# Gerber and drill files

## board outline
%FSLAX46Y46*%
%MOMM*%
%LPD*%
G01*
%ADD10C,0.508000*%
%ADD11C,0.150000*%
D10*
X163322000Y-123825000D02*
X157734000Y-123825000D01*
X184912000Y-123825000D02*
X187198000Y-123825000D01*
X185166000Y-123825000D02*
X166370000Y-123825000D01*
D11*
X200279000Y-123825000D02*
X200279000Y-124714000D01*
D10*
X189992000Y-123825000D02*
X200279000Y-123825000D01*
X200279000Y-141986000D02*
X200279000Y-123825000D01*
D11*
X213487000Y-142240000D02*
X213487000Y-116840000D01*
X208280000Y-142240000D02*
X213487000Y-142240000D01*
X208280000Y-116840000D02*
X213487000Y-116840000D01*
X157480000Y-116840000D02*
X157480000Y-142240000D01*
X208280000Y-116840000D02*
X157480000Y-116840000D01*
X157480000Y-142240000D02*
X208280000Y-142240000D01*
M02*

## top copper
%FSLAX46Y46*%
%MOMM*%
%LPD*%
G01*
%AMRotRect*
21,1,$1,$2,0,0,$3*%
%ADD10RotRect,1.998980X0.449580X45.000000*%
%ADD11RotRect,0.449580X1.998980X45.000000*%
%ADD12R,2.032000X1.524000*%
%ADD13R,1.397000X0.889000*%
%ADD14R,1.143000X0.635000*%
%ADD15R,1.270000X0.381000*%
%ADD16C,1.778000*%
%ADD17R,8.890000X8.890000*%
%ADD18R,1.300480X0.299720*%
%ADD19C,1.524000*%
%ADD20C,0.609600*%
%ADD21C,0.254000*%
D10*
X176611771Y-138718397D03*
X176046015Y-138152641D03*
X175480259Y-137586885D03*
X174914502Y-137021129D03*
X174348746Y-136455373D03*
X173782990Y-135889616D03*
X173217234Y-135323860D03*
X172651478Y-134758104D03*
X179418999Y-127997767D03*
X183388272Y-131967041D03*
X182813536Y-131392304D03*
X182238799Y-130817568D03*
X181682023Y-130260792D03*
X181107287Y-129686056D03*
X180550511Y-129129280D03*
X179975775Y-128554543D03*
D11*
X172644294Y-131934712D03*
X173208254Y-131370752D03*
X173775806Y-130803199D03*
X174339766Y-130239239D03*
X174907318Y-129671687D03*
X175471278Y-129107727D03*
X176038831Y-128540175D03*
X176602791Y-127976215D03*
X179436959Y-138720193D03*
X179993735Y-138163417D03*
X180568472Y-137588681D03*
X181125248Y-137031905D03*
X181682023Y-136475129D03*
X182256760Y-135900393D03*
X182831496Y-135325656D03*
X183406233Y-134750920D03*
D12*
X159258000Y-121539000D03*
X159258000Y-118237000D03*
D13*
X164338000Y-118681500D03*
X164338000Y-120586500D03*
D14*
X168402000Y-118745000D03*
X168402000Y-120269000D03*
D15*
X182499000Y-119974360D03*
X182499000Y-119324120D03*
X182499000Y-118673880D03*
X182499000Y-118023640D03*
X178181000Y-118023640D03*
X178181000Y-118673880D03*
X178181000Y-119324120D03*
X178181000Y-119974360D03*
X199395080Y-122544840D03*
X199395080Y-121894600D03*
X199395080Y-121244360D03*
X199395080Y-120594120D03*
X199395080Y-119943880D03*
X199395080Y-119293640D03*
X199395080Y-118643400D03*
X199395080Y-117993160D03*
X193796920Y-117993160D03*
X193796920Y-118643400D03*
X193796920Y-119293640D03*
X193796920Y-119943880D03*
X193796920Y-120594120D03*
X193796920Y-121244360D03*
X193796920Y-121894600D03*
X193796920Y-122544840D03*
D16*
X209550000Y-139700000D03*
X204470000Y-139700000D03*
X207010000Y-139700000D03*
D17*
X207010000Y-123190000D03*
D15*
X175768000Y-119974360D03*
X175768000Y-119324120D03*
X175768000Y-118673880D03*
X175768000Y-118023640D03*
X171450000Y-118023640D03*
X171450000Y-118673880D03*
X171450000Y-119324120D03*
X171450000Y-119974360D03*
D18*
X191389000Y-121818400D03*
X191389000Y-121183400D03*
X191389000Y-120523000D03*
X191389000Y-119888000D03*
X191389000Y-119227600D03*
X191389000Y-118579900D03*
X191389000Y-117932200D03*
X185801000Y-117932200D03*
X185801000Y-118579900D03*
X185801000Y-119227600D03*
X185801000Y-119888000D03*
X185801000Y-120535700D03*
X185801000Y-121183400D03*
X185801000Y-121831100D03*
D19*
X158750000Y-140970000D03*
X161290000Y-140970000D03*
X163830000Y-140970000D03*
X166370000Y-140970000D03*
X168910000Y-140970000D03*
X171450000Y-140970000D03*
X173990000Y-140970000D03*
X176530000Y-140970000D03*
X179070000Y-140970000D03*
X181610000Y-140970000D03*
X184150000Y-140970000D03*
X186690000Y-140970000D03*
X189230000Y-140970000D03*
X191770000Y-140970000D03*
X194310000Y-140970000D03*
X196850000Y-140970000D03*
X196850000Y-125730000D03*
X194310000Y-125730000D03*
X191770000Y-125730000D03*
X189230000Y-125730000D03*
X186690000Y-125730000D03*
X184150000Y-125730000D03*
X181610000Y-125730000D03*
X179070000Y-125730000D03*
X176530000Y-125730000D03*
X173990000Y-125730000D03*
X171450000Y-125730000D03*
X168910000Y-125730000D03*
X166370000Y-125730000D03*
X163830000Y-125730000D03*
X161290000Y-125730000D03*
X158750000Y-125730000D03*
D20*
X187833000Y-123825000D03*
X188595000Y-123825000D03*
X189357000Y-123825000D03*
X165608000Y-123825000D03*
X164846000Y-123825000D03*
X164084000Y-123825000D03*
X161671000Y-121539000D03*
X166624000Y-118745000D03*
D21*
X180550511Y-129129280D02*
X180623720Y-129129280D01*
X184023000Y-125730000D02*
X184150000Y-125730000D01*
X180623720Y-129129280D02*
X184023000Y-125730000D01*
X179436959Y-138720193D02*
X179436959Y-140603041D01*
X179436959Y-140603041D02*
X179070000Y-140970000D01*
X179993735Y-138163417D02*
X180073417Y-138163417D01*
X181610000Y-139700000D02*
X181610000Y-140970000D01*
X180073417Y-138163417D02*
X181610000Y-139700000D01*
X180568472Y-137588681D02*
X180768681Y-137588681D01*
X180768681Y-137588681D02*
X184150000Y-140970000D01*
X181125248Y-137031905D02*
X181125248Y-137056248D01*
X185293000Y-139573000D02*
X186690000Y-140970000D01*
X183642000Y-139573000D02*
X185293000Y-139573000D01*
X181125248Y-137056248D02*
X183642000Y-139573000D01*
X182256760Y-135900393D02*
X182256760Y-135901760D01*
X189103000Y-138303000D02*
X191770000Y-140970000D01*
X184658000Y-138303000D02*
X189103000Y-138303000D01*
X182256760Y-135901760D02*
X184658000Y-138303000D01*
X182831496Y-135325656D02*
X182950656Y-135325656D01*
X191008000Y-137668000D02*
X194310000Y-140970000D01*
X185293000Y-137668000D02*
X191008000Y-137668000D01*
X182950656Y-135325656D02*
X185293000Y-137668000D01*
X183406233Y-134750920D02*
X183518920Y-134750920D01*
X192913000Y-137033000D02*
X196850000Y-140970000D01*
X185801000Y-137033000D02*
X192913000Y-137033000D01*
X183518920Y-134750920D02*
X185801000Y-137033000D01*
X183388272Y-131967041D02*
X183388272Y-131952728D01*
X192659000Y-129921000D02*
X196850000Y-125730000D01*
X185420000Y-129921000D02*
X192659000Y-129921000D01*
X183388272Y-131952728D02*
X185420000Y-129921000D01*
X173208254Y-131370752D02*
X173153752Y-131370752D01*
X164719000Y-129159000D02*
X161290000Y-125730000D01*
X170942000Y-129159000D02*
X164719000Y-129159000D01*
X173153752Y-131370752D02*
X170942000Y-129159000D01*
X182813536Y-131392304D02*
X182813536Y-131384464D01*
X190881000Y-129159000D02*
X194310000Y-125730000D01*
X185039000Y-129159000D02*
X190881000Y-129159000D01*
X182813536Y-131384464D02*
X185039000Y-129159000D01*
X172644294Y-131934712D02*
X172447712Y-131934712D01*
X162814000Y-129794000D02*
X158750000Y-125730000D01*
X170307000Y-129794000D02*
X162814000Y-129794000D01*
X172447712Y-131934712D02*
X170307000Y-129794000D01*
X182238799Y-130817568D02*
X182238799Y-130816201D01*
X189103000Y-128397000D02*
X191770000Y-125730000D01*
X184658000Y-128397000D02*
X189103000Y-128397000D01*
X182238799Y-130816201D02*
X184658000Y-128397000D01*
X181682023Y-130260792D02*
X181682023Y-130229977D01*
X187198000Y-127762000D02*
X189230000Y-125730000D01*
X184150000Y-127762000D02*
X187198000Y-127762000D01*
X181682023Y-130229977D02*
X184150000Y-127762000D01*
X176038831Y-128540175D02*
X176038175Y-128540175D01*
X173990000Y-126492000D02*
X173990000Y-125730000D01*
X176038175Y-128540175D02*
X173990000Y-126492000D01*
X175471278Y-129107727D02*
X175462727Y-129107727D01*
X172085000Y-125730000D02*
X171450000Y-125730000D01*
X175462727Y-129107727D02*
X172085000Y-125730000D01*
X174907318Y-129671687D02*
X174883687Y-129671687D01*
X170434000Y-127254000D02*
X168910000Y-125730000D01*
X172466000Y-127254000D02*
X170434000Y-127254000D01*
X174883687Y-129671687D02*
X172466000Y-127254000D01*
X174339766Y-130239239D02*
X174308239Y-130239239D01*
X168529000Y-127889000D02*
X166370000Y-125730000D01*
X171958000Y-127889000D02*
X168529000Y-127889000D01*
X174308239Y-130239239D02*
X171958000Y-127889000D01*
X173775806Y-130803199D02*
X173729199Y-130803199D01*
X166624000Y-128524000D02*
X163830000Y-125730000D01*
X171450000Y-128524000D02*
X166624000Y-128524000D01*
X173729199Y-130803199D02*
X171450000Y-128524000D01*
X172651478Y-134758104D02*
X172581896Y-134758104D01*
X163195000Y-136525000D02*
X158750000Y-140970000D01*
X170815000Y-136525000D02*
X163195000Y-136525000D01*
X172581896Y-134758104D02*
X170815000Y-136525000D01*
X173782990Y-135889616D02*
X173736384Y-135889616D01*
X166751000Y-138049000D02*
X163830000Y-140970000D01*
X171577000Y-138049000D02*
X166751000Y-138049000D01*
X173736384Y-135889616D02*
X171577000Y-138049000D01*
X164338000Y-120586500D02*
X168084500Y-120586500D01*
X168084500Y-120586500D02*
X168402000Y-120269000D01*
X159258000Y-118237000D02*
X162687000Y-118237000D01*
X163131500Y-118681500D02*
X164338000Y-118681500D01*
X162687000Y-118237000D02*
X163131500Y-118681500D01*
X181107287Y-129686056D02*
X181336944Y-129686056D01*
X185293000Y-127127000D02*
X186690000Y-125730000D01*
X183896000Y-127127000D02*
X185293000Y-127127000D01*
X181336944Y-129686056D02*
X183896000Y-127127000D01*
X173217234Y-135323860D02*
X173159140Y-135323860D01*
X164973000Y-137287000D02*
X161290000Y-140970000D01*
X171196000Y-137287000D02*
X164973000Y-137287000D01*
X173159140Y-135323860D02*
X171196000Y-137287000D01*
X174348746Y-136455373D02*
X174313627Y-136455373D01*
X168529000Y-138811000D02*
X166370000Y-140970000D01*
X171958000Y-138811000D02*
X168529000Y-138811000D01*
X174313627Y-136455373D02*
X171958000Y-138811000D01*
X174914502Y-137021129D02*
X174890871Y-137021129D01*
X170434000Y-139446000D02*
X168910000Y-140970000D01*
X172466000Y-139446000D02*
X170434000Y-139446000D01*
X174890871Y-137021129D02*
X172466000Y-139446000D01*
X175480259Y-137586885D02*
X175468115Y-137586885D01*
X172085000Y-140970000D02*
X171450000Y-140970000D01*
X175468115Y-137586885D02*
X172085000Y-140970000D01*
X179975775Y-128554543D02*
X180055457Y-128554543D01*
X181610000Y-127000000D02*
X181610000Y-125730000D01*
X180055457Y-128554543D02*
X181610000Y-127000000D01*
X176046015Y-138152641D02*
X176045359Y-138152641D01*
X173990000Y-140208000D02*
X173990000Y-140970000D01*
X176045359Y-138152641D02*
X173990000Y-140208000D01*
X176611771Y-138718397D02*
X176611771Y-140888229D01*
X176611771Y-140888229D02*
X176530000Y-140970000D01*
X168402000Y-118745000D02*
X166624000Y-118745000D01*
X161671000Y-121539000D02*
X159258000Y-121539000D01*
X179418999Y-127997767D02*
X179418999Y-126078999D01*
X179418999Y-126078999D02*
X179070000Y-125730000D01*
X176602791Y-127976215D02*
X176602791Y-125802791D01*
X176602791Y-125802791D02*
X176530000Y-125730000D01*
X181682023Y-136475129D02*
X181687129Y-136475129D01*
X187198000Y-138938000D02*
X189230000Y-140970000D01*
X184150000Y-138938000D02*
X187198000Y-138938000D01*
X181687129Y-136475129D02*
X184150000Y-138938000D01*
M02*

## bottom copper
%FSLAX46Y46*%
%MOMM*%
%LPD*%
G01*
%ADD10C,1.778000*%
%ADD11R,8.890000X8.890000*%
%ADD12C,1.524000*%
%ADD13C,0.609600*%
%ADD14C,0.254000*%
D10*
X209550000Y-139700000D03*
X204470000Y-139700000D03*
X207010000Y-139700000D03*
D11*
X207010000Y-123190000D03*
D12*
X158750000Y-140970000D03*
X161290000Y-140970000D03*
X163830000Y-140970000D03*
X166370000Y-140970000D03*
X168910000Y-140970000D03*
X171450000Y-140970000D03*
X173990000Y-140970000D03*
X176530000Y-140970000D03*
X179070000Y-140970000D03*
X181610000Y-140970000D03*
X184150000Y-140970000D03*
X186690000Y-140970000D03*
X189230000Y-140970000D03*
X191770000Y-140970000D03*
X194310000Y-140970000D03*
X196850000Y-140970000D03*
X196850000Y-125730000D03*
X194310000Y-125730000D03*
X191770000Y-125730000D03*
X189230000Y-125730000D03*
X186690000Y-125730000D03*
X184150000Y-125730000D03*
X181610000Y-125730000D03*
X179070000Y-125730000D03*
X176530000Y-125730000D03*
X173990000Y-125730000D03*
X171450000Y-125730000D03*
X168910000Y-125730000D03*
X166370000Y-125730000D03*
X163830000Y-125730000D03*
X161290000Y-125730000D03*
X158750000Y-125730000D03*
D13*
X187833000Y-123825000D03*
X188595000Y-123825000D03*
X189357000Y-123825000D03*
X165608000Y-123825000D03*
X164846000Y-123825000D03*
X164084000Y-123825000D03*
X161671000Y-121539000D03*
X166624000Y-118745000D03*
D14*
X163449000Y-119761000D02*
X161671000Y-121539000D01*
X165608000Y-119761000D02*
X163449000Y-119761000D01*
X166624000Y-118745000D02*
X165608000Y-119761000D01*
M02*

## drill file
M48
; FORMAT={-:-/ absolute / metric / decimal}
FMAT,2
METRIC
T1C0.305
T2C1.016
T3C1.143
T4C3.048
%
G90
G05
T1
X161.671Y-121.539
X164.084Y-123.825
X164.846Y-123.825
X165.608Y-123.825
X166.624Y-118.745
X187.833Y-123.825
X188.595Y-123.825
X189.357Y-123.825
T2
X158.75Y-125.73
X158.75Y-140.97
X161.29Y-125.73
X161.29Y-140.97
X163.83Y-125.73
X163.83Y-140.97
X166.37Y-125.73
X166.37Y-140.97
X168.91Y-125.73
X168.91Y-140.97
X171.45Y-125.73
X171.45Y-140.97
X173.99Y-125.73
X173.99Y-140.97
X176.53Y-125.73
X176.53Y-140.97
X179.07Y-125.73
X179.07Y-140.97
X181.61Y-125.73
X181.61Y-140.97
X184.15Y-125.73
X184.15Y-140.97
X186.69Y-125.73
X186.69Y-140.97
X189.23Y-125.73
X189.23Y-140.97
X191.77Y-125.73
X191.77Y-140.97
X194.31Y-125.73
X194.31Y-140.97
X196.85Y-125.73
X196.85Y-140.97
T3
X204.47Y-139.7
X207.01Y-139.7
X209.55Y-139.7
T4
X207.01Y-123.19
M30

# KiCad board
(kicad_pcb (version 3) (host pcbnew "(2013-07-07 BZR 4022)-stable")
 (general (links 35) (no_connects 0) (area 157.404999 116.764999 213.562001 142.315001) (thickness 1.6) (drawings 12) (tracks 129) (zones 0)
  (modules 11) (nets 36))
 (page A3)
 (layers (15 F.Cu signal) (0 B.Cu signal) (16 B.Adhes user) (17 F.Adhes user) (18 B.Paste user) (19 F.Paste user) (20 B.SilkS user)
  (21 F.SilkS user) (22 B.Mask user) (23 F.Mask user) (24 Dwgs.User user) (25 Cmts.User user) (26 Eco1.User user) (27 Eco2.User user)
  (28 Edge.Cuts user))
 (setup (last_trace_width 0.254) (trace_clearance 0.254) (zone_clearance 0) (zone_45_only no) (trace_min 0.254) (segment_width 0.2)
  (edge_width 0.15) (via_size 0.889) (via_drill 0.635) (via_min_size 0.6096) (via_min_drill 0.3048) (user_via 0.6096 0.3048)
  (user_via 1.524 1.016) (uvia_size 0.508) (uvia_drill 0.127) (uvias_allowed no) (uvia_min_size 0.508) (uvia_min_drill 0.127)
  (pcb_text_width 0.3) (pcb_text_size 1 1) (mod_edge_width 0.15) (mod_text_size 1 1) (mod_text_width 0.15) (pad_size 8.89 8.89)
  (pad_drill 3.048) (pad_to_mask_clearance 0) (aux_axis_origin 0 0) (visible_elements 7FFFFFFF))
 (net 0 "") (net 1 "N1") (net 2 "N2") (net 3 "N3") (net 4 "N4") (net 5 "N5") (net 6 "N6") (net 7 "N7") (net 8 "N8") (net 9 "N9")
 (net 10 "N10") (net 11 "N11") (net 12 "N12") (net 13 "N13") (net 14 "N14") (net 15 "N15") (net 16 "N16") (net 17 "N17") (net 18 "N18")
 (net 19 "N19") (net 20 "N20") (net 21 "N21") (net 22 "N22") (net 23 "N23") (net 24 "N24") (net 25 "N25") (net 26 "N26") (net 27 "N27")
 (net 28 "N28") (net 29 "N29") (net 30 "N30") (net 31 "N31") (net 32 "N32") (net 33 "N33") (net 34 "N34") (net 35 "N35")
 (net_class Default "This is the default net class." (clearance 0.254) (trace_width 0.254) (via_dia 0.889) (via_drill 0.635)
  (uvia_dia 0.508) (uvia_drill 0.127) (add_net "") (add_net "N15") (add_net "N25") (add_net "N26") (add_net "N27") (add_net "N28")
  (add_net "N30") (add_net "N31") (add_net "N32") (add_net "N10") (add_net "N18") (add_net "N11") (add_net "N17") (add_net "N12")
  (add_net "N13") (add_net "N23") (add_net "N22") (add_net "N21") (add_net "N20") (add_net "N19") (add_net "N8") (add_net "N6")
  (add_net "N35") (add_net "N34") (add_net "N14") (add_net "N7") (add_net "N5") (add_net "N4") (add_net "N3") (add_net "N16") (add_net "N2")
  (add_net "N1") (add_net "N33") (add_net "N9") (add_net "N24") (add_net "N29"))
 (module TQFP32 (layer F.Cu) (at 178.054 133.35 45)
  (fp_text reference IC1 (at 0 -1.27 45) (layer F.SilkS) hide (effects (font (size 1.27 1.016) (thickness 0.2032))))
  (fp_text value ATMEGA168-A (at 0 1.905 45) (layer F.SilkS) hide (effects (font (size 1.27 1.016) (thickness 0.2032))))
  (pad 8 smd rect (at -4.81584 2.77622 45) (size 1.99898 0.44958) (layers F.Cu F.Paste F.Mask) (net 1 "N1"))
  (pad 7 smd rect (at -4.81584 1.97612 45) (size 1.99898 0.44958) (layers F.Cu F.Paste F.Mask) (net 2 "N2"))
  (pad 6 smd rect (at -4.81584 1.17602 45) (size 1.99898 0.44958) (layers F.Cu F.Paste F.Mask) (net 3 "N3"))
  (pad 5 smd rect (at -4.81584 0.37592 45) (size 1.99898 0.44958) (layers F.Cu F.Paste F.Mask) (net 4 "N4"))
  (pad 4 smd rect (at -4.81584 -0.42418 45) (size 1.99898 0.44958) (layers F.Cu F.Paste F.Mask) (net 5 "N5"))
  (pad 3 smd rect (at -4.81584 -1.22428 45) (size 1.99898 0.44958) (layers F.Cu F.Paste F.Mask) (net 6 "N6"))
  (pad 2 smd rect (at -4.81584 -2.02438 45) (size 1.99898 0.44958) (layers F.Cu F.Paste F.Mask) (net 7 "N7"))
  (pad 1 smd rect (at -4.81584 -2.82448 45) (size 1.99898 0.44958) (layers F.Cu F.Paste F.Mask) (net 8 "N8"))
  (pad 24 smd rect (at 4.7498 -2.8194 45) (size 1.99898 0.44958) (layers F.Cu F.Paste F.Mask) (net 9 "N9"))
  (pad 17 smd rect (at 4.7498 2.794 45) (size 1.99898 0.44958) (layers F.Cu F.Paste F.Mask) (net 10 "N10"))
  (pad 18 smd rect (at 4.7498 1.9812 45) (size 1.99898 0.44958) (layers F.Cu F.Paste F.Mask) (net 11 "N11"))
  (pad 19 smd rect (at 4.7498 1.1684 45) (size 1.99898 0.44958) (layers F.Cu F.Paste F.Mask) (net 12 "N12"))
  (pad 20 smd rect (at 4.7498 0.381 45) (size 1.99898 0.44958) (layers F.Cu F.Paste F.Mask) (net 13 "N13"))
  (pad 21 smd rect (at 4.7498 -0.4318 45) (size 1.99898 0.44958) (layers F.Cu F.Paste F.Mask) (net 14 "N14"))
  (pad 22 smd rect (at 4.7498 -1.2192 45) (size 1.99898 0.44958) (layers F.Cu F.Paste F.Mask) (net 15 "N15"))
  (pad 23 smd rect (at 4.7498 -2.032 45) (size 1.99898 0.44958) (layers F.Cu F.Paste F.Mask) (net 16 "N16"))
  (pad 32 smd rect (at -2.82448 -4.826 45) (size 0.44958 1.99898) (layers F.Cu F.Paste F.Mask) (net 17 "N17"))
  (pad 31 smd rect (at -2.02692 -4.826 45) (size 0.44958 1.99898) (layers F.Cu F.Paste F.Mask) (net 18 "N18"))
  (pad 30 smd rect (at -1.22428 -4.826 45) (size 0.44958 1.99898) (layers F.Cu F.Paste F.Mask) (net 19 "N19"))
  (pad 29 smd rect (at -0.42672 -4.826 45) (size 0.44958 1.99898) (layers F.Cu F.Paste F.Mask) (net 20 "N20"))
  (pad 28 smd rect (at 0.37592 -4.826 45) (size 0.44958 1.99898) (layers F.Cu F.Paste F.Mask) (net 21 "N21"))
  (pad 27 smd rect (at 1.17348 -4.826 45) (size 0.44958 1.99898) (layers F.Cu F.Paste F.Mask) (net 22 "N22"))
  (pad 26 smd rect (at 1.97612 -4.826 45) (size 0.44958 1.99898) (layers F.Cu F.Paste F.Mask) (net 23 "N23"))
  (pad 25 smd rect (at 2.77368 -4.826 45) (size 0.44958 1.99898) (layers F.Cu F.Paste F.Mask) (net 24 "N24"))
  (pad 9 smd rect (at -2.8194 4.7752 45) (size 0.44958 1.99898) (layers F.Cu F.Paste F.Mask) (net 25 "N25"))
  (pad 10 smd rect (at -2.032 4.7752 45) (size 0.44958 1.99898) (layers F.Cu F.Paste F.Mask) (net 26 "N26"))
  (pad 11 smd rect (at -1.2192 4.7752 45) (size 0.44958 1.99898) (layers F.Cu F.Paste F.Mask) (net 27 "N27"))
  (pad 12 smd rect (at -0.4318 4.7752 45) (size 0.44958 1.99898) (layers F.Cu F.Paste F.Mask) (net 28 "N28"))
  (pad 13 smd rect (at 0.3556 4.7752 45) (size 0.44958 1.99898) (layers F.Cu F.Paste F.Mask) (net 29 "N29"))
  (pad 14 smd rect (at 1.1684 4.7752 45) (size 0.44958 1.99898) (layers F.Cu F.Paste F.Mask) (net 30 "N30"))
  (pad 15 smd rect (at 1.9812 4.7752 45) (size 0.44958 1.99898) (layers F.Cu F.Paste F.Mask) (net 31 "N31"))
  (pad 16 smd rect (at 2.794 4.7752 45) (size 0.44958 1.99898) (layers F.Cu F.Paste F.Mask) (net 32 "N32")))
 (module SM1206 (layer F.Cu) (at 159.258 119.888 90)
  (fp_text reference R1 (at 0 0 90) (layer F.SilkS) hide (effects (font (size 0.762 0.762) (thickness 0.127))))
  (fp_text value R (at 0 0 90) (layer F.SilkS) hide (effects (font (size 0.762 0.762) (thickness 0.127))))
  (pad 1 smd rect (at -1.651 0 90) (size 1.524 2.032) (layers F.Cu F.Paste F.Mask) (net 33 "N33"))
  (pad 2 smd rect (at 1.651 0 90) (size 1.524 2.032) (layers F.Cu F.Paste F.Mask) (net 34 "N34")))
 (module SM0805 (layer F.Cu) (at 164.338 119.634 270)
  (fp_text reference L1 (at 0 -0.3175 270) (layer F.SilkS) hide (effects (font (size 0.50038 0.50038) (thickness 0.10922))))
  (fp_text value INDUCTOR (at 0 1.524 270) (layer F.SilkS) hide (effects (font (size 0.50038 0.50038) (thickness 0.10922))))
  (pad 1 smd rect (at -0.9525 0 270) (size 0.889 1.397) (layers F.Cu F.Paste F.Mask) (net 34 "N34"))
  (pad 2 smd rect (at 0.9525 0 270) (size 0.889 1.397) (layers F.Cu F.Paste F.Mask) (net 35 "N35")))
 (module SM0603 (layer F.Cu) (at 168.402 119.507 270)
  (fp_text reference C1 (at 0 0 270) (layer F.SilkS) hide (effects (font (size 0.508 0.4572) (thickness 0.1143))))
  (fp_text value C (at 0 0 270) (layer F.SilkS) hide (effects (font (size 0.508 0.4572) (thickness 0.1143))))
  (pad 1 smd rect (at -0.762 0 270) (size 0.635 1.143) (layers F.Cu F.Paste F.Mask) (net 33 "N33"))
  (pad 2 smd rect (at 0.762 0 270) (size 0.635 1.143) (layers F.Cu F.Paste F.Mask) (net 35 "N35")))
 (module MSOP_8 (layer F.Cu) (at 180.34 118.999 90)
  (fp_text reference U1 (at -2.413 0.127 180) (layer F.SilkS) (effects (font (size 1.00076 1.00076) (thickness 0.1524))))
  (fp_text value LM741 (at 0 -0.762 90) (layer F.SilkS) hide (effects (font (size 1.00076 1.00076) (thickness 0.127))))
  (pad 1 smd rect (at -0.97536 2.159 90) (size 0.381 1.27) (layers F.Cu F.Paste F.Mask))
  (pad 2 smd rect (at -0.32512 2.159 90) (size 0.381 1.27) (layers F.Cu F.Paste F.Mask))
  (pad 3 smd rect (at 0.32512 2.159 90) (size 0.381 1.27) (layers F.Cu F.Paste F.Mask))
  (pad 4 smd rect (at 0.97536 2.159 90) (size 0.381 1.27) (layers F.Cu F.Paste F.Mask))
  (pad 5 smd rect (at 0.97536 -2.159 90) (size 0.381 1.27) (layers F.Cu F.Paste F.Mask))
  (pad 6 smd rect (at 0.32512 -2.159 90) (size 0.381 1.27) (layers F.Cu F.Paste F.Mask))
  (pad 7 smd rect (at -0.32512 -2.159 90) (size 0.381 1.27) (layers F.Cu F.Paste F.Mask))
  (pad 8 smd rect (at -0.97536 -2.159 90) (size 0.381 1.27) (layers F.Cu F.Paste F.Mask)))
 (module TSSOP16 (layer F.Cu) (at 196.596 120.269 90)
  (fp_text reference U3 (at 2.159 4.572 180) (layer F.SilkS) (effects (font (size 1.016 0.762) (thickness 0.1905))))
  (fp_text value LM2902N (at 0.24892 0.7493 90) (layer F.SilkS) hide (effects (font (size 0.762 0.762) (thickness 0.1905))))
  (pad 1 smd rect (at -2.27584 2.79908 90) (size 0.381 1.27) (layers F.Cu F.Paste F.Mask))
  (pad 2 smd rect (at -1.6256 2.79908 90) (size 0.381 1.27) (layers F.Cu F.Paste F.Mask))
  (pad 3 smd rect (at -0.97536 2.79908 90) (size 0.381 1.27) (layers F.Cu F.Paste F.Mask))
  (pad 4 smd rect (at -0.32512 2.79908 90) (size 0.381 1.27) (layers F.Cu F.Paste F.Mask))
  (pad 5 smd rect (at 0.32512 2.79908 90) (size 0.381 1.27) (layers F.Cu F.Paste F.Mask))
  (pad 6 smd rect (at 0.97536 2.79908 90) (size 0.381 1.27) (layers F.Cu F.Paste F.Mask))
  (pad 7 smd rect (at 1.6256 2.79908 90) (size 0.381 1.27) (layers F.Cu F.Paste F.Mask))
  (pad 8 smd rect (at 2.27584 2.79908 90) (size 0.381 1.27) (layers F.Cu F.Paste F.Mask))
  (pad 9 smd rect (at 2.27584 -2.79908 90) (size 0.381 1.27) (layers F.Cu F.Paste F.Mask))
  (pad 10 smd rect (at 1.6256 -2.79908 90) (size 0.381 1.27) (layers F.Cu F.Paste F.Mask))
  (pad 11 smd rect (at 0.97536 -2.79908 90) (size 0.381 1.27) (layers F.Cu F.Paste F.Mask))
  (pad 12 smd rect (at 0.32512 -2.79908 90) (size 0.381 1.27) (layers F.Cu F.Paste F.Mask))
  (pad 13 smd rect (at -0.32512 -2.79908 90) (size 0.381 1.27) (layers F.Cu F.Paste F.Mask))
  (pad 14 smd rect (at -0.97536 -2.79908 90) (size 0.381 1.27) (layers F.Cu F.Paste F.Mask))
  (pad 15 smd rect (at -1.6256 -2.79908 90) (size 0.381 1.27) (layers F.Cu F.Paste F.Mask))
  (pad 16 smd rect (at -2.27584 -2.79908 90) (size 0.381 1.27) (layers F.Cu F.Paste F.Mask)))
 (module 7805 (layer F.Cu) (at 207.01 139.7 90)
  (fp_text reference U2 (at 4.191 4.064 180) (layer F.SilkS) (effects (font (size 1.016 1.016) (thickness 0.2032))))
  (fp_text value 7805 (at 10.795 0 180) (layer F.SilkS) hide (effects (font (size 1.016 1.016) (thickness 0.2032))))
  (pad VO thru_hole circle (at 0 2.54 90) (size 1.778 1.778) (drill 1.143) (layers *.Cu *.Mask F.SilkS))
  (pad VI thru_hole circle (at 0 -2.54 90) (size 1.778 1.778) (drill 1.143) (layers *.Cu *.Mask F.SilkS))
  (pad GND thru_hole circle (at 0 0 90) (size 1.778 1.778) (drill 1.143) (layers *.Cu *.Mask F.SilkS))
  (pad GND thru_hole rect (at 16.51 0 90) (size 8.89 8.89) (drill 3.048) (layers *.Cu *.SilkS *.Mask)))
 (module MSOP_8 (layer F.Cu) (at 173.609 118.999 90)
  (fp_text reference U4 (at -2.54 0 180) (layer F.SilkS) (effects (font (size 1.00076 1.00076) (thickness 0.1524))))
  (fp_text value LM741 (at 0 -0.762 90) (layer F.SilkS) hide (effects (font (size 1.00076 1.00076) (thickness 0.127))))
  (pad 1 smd rect (at -0.97536 2.159 90) (size 0.381 1.27) (layers F.Cu F.Paste F.Mask))
  (pad 2 smd rect (at -0.32512 2.159 90) (size 0.381 1.27) (layers F.Cu F.Paste F.Mask))
  (pad 3 smd rect (at 0.32512 2.159 90) (size 0.381 1.27) (layers F.Cu F.Paste F.Mask))
  (pad 4 smd rect (at 0.97536 2.159 90) (size 0.381 1.27) (layers F.Cu F.Paste F.Mask))
  (pad 5 smd rect (at 0.97536 -2.159 90) (size 0.381 1.27) (layers F.Cu F.Paste F.Mask))
  (pad 6 smd rect (at 0.32512 -2.159 90) (size 0.381 1.27) (layers F.Cu F.Paste F.Mask))
  (pad 7 smd rect (at -0.32512 -2.159 90) (size 0.381 1.27) (layers F.Cu F.Paste F.Mask))
  (pad 8 smd rect (at -0.97536 -2.159 90) (size 0.381 1.27) (layers F.Cu F.Paste F.Mask)))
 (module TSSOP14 (layer F.Cu) (at 188.595 119.888 90)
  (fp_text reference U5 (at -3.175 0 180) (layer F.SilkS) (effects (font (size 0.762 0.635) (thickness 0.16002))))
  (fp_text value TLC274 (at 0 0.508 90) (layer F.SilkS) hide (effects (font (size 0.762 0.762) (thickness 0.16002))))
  (pad 1 smd rect (at -1.9304 2.794 90) (size 0.29972 1.30048) (layers F.Cu F.Paste F.Mask))
  (pad 2 smd rect (at -1.2954 2.794 90) (size 0.29972 1.30048) (layers F.Cu F.Paste F.Mask))
  (pad 3 smd rect (at -0.635 2.794 90) (size 0.29972 1.30048) (layers F.Cu F.Paste F.Mask))
  (pad 4 smd rect (at 0 2.794 90) (size 0.29972 1.30048) (layers F.Cu F.Paste F.Mask))
  (pad 5 smd rect (at 0.6604 2.794 90) (size 0.29972 1.30048) (layers F.Cu F.Paste F.Mask))
  (pad 6 smd rect (at 1.3081 2.794 90) (size 0.29972 1.30048) (layers F.Cu F.Paste F.Mask))
  (pad 7 smd rect (at 1.9558 2.794 90) (size 0.29972 1.30048) (layers F.Cu F.Paste F.Mask))
  (pad 8 smd rect (at 1.9558 -2.794 90) (size 0.29972 1.30048) (layers F.Cu F.Paste F.Mask))
  (pad 9 smd rect (at 1.3081 -2.794 90) (size 0.29972 1.30048) (layers F.Cu F.Paste F.Mask))
  (pad 10 smd rect (at 0.6604 -2.794 90) (size 0.29972 1.30048) (layers F.Cu F.Paste F.Mask))
  (pad 11 smd rect (at 0 -2.794 90) (size 0.29972 1.30048) (layers F.Cu F.Paste F.Mask))
  (pad 12 smd rect (at -0.6477 -2.794 90) (size 0.29972 1.30048) (layers F.Cu F.Paste F.Mask))
  (pad 13 smd rect (at -1.2954 -2.794 90) (size 0.29972 1.30048) (layers F.Cu F.Paste F.Mask))
  (pad 14 smd rect (at -1.9431 -2.794 90) (size 0.29972 1.30048) (layers F.Cu F.Paste F.Mask)))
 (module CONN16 (layer F.Cu) (at 158.75 140.97 90)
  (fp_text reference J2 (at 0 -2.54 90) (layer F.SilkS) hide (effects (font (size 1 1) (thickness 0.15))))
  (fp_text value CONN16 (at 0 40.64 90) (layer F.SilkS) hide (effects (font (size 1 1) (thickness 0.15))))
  (pad 1 thru_hole circle (at 0 0 90) (size 1.524 1.524) (drill 1.016) (layers *.Cu *.Mask F.SilkS) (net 8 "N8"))
  (pad 2 thru_hole circle (at 0 2.54 90) (size 1.524 1.524) (drill 1.016) (layers *.Cu *.Mask F.SilkS) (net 7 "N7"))
  (pad 3 thru_hole circle (at 0 5.08 90) (size 1.524 1.524) (drill 1.016) (layers *.Cu *.Mask F.SilkS) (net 6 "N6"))
  (pad 4 thru_hole circle (at 0 7.62 90) (size 1.524 1.524) (drill 1.016) (layers *.Cu *.Mask F.SilkS) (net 5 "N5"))
  (pad 5 thru_hole circle (at 0 10.16 90) (size 1.524 1.524) (drill 1.016) (layers *.Cu *.Mask F.SilkS) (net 4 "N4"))
  (pad 6 thru_hole circle (at 0 12.7 90) (size 1.524 1.524) (drill 1.016) (layers *.Cu *.Mask F.SilkS) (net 3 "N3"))
  (pad 7 thru_hole circle (at 0 15.24 90) (size 1.524 1.524) (drill 1.016) (layers *.Cu *.Mask F.SilkS) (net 2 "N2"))
  (pad 8 thru_hole circle (at 0 17.78 90) (size 1.524 1.524) (drill 1.016) (layers *.Cu *.Mask F.SilkS) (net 1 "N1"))
  (pad 9 thru_hole circle (at 0 20.32 90) (size 1.524 1.524) (drill 1.016) (layers *.Cu *.Mask F.SilkS) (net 25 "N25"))
  (pad 10 thru_hole circle (at 0 22.86 90) (size 1.524 1.524) (drill 1.016) (layers *.Cu *.Mask F.SilkS) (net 26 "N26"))
  (pad 11 thru_hole circle (at 0 25.4 90) (size 1.524 1.524) (drill 1.016) (layers *.Cu *.Mask F.SilkS) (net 27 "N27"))
  (pad 12 thru_hole circle (at 0 27.94 90) (size 1.524 1.524) (drill 1.016) (layers *.Cu *.Mask F.SilkS) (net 28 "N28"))
  (pad 13 thru_hole circle (at 0 30.48 90) (size 1.524 1.524) (drill 1.016) (layers *.Cu *.Mask F.SilkS) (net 29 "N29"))
  (pad 14 thru_hole circle (at 0 33.02 90) (size 1.524 1.524) (drill 1.016) (layers *.Cu *.Mask F.SilkS) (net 30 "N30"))
  (pad 15 thru_hole circle (at 0 35.56 90) (size 1.524 1.524) (drill 1.016) (layers *.Cu *.Mask F.SilkS) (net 31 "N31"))
  (pad 16 thru_hole circle (at 0 38.1 90) (size 1.524 1.524) (drill 1.016) (layers *.Cu *.Mask F.SilkS) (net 32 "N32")))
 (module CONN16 (layer F.Cu) (at 196.85 125.73 270)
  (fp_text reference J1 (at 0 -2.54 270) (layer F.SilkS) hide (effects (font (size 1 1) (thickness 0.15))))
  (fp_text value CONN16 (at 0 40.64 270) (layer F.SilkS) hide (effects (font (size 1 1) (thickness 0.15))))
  (pad 1 thru_hole circle (at 0 0 270) (size 1.524 1.524) (drill 1.016) (layers *.Cu *.Mask F.SilkS) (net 10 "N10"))
  (pad 2 thru_hole circle (at 0 2.54 270) (size 1.524 1.524) (drill 1.016) (layers *.Cu *.Mask F.SilkS) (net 11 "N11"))
  (pad 3 thru_hole circle (at 0 5.08 270) (size 1.524 1.524) (drill 1.016) (layers *.Cu *.Mask F.SilkS) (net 12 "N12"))
  (pad 4 thru_hole circle (at 0 7.62 270) (size 1.524 1.524) (drill 1.016) (layers *.Cu *.Mask F.SilkS) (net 13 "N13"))
  (pad 5 thru_hole circle (at 0 10.16 270) (size 1.524 1.524) (drill 1.016) (layers *.Cu *.Mask F.SilkS) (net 14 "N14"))
  (pad 6 thru_hole circle (at 0 12.7 270) (size 1.524 1.524) (drill 1.016) (layers *.Cu *.Mask F.SilkS) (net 15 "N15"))
  (pad 7 thru_hole circle (at 0 15.24 270) (size 1.524 1.524) (drill 1.016) (layers *.Cu *.Mask F.SilkS) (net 16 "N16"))
  (pad 8 thru_hole circle (at 0 17.78 270) (size 1.524 1.524) (drill 1.016) (layers *.Cu *.Mask F.SilkS) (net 9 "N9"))
  (pad 9 thru_hole circle (at 0 20.32 270) (size 1.524 1.524) (drill 1.016) (layers *.Cu *.Mask F.SilkS) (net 24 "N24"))
  (pad 10 thru_hole circle (at 0 22.86 270) (size 1.524 1.524) (drill 1.016) (layers *.Cu *.Mask F.SilkS) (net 23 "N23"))
  (pad 11 thru_hole circle (at 0 25.4 270) (size 1.524 1.524) (drill 1.016) (layers *.Cu *.Mask F.SilkS) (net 22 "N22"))
  (pad 12 thru_hole circle (at 0 27.94 270) (size 1.524 1.524) (drill 1.016) (layers *.Cu *.Mask F.SilkS) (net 21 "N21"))
  (pad 13 thru_hole circle (at 0 30.48 270) (size 1.524 1.524) (drill 1.016) (layers *.Cu *.Mask F.SilkS) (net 20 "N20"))
  (pad 14 thru_hole circle (at 0 33.02 270) (size 1.524 1.524) (drill 1.016) (layers *.Cu *.Mask F.SilkS) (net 19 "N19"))
  (pad 15 thru_hole circle (at 0 35.56 270) (size 1.524 1.524) (drill 1.016) (layers *.Cu *.Mask F.SilkS) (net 18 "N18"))
  (pad 16 thru_hole circle (at 0 38.1 270) (size 1.524 1.524) (drill 1.016) (layers *.Cu *.Mask F.SilkS) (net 17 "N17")))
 (gr_line (start 163.322 123.825) (end 157.734 123.825) (angle 90) (layer Edge.Cuts) (width 0.508))
 (gr_line (start 184.912 123.825) (end 187.198 123.825) (angle 90) (layer Edge.Cuts) (width 0.508))
 (gr_line (start 185.166 123.825) (end 166.37 123.825) (angle 90) (layer Edge.Cuts) (width 0.508))
 (gr_line (start 200.279 123.825) (end 200.279 124.714) (angle 90) (layer Edge.Cuts) (width 0.15))
 (gr_line (start 189.992 123.825) (end 200.279 123.825) (angle 90) (layer Edge.Cuts) (width 0.508))
 (gr_line (start 200.279 141.986) (end 200.279 123.825) (angle 90) (layer Edge.Cuts) (width 0.508))
 (gr_line (start 213.487 142.24) (end 213.487 116.84) (angle 90) (layer Edge.Cuts) (width 0.15))
 (gr_line (start 208.28 142.24) (end 213.487 142.24) (angle 90) (layer Edge.Cuts) (width 0.15))
 (gr_line (start 208.28 116.84) (end 213.487 116.84) (angle 90) (layer Edge.Cuts) (width 0.15))
 (gr_line (start 157.48 116.84) (end 157.48 142.24) (angle 90) (layer Edge.Cuts) (width 0.15))
 (gr_line (start 208.28 116.84) (end 157.48 116.84) (angle 90) (layer Edge.Cuts) (width 0.15))
 (gr_line (start 157.48 142.24) (end 208.28 142.24) (angle 90) (layer Edge.Cuts) (width 0.15))
 (via (at 187.833 123.825) (size 0.6096) (drill 0.3048) (layers F.Cu B.Cu) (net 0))
 (via (at 188.595 123.825) (size 0.6096) (drill 0.3048) (layers F.Cu B.Cu) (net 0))
 (via (at 189.357 123.825) (size 0.6096) (drill 0.3048) (layers F.Cu B.Cu) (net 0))
 (via (at 165.608 123.825) (size 0.6096) (drill 0.3048) (layers F.Cu B.Cu) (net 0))
 (via (at 164.846 123.825) (size 0.6096) (drill 0.3048) (layers F.Cu B.Cu) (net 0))
 (via (at 164.084 123.825) (size 0.6096) (drill 0.3048) (layers F.Cu B.Cu) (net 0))
 (segment (start 180.550511 129.12928) (end 180.62372 129.12928) (width 0.254) (layer F.Cu) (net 15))
 (segment (start 184.023 125.73) (end 184.15 125.73) (width 0.254) (layer F.Cu) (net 15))
 (segment (start 180.62372 129.12928) (end 184.023 125.73) (width 0.254) (layer F.Cu) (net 15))
 (segment (start 179.436959 138.720193) (end 179.436959 140.603041) (width 0.254) (layer F.Cu) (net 25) (status 10))
 (segment (start 179.436959 140.603041) (end 179.07 140.97) (width 0.254) (layer F.Cu) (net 25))
 (segment (start 179.993735 138.163417) (end 180.073417 138.163417) (width 0.254) (layer F.Cu) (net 26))
 (segment (start 181.61 139.7) (end 181.61 140.97) (width 0.254) (layer F.Cu) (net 26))
 (segment (start 180.073417 138.163417) (end 181.61 139.7) (width 0.254) (layer F.Cu) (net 26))
 (segment (start 180.568472 137.588681) (end 180.768681 137.588681) (width 0.254) (layer F.Cu) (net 27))
 (segment (start 180.768681 137.588681) (end 184.15 140.97) (width 0.254) (layer F.Cu) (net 27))
 (segment (start 181.125248 137.031905) (end 181.125248 137.056248) (width 0.254) (layer F.Cu) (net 28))
 (segment (start 185.293 139.573) (end 186.69 140.97) (width 0.254) (layer F.Cu) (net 28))
 (segment (start 183.642 139.573) (end 185.293 139.573) (width 0.254) (layer F.Cu) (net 28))
 (segment (start 181.125248 137.056248) (end 183.642 139.573) (width 0.254) (layer F.Cu) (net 28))
 (segment (start 182.25676 135.900393) (end 182.25676 135.90176) (width 0.254) (layer F.Cu) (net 30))
 (segment (start 189.103 138.303) (end 191.77 140.97) (width 0.254) (layer F.Cu) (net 30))
 (segment (start 184.658 138.303) (end 189.103 138.303) (width 0.254) (layer F.Cu) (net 30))
 (segment (start 182.25676 135.90176) (end 184.658 138.303) (width 0.254) (layer F.Cu) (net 30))
 (segment (start 182.831496 135.325656) (end 182.950656 135.325656) (width 0.254) (layer F.Cu) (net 31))
 (segment (start 191.008 137.668) (end 194.31 140.97) (width 0.254) (layer F.Cu) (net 31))
 (segment (start 185.293 137.668) (end 191.008 137.668) (width 0.254) (layer F.Cu) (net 31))
 (segment (start 182.950656 135.325656) (end 185.293 137.668) (width 0.254) (layer F.Cu) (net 31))
 (segment (start 183.406233 134.75092) (end 183.51892 134.75092) (width 0.254) (layer F.Cu) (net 32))
 (segment (start 192.913 137.033) (end 196.85 140.97) (width 0.254) (layer F.Cu) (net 32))
 (segment (start 185.801 137.033) (end 192.913 137.033) (width 0.254) (layer F.Cu) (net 32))
 (segment (start 183.51892 134.75092) (end 185.801 137.033) (width 0.254) (layer F.Cu) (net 32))
 (segment (start 183.388272 131.967041) (end 183.388272 131.952728) (width 0.254) (layer F.Cu) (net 10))
 (segment (start 192.659 129.921) (end 196.85 125.73) (width 0.254) (layer F.Cu) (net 10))
 (segment (start 185.42 129.921) (end 192.659 129.921) (width 0.254) (layer F.Cu) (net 10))
 (segment (start 183.388272 131.952728) (end 185.42 129.921) (width 0.254) (layer F.Cu) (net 10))
 (segment (start 173.208254 131.370752) (end 173.153752 131.370752) (width 0.254) (layer F.Cu) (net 18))
 (segment (start 164.719 129.159) (end 161.29 125.73) (width 0.254) (layer F.Cu) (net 18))
 (segment (start 170.942 129.159) (end 164.719 129.159) (width 0.254) (layer F.Cu) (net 18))
 (segment (start 173.153752 131.370752) (end 170.942 129.159) (width 0.254) (layer F.Cu) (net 18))
 (segment (start 182.813536 131.392304) (end 182.813536 131.384464) (width 0.254) (layer F.Cu) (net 11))
 (segment (start 190.881 129.159) (end 194.31 125.73) (width 0.254) (layer F.Cu) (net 11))
 (segment (start 185.039 129.159) (end 190.881 129.159) (width 0.254) (layer F.Cu) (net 11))
 (segment (start 182.813536 131.384464) (end 185.039 129.159) (width 0.254) (layer F.Cu) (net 11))
 (segment (start 172.644294 131.934712) (end 172.447712 131.934712) (width 0.254) (layer F.Cu) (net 17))
 (segment (start 162.814 129.794) (end 158.75 125.73) (width 0.254) (layer F.Cu) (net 17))
 (segment (start 170.307 129.794) (end 162.814 129.794) (width 0.254) (layer F.Cu) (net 17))
 (segment (start 172.447712 131.934712) (end 170.307 129.794) (width 0.254) (layer F.Cu) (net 17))
 (segment (start 182.238799 130.817568) (end 182.238799 130.816201) (width 0.254) (layer F.Cu) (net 12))
 (segment (start 189.103 128.397) (end 191.77 125.73) (width 0.254) (layer F.Cu) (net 12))
 (segment (start 184.658 128.397) (end 189.103 128.397) (width 0.254) (layer F.Cu) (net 12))
 (segment (start 182.238799 130.816201) (end 184.658 128.397) (width 0.254) (layer F.Cu) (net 12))
 (segment (start 181.682023 130.260792) (end 181.682023 130.229977) (width 0.254) (layer F.Cu) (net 13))
 (segment (start 187.198 127.762) (end 189.23 125.73) (width 0.254) (layer F.Cu) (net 13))
 (segment (start 184.15 127.762) (end 187.198 127.762) (width 0.254) (layer F.Cu) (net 13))
 (segment (start 181.682023 130.229977) (end 184.15 127.762) (width 0.254) (layer F.Cu) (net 13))
 (segment (start 176.038831 128.540175) (end 176.038175 128.540175) (width 0.254) (layer F.Cu) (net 23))
 (segment (start 173.99 126.492) (end 173.99 125.73) (width 0.254) (layer F.Cu) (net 23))
 (segment (start 176.038175 128.540175) (end 173.99 126.492) (width 0.254) (layer F.Cu) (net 23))
 (segment (start 175.471278 129.107727) (end 175.462727 129.107727) (width 0.254) (layer F.Cu) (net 22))
 (segment (start 172.085 125.73) (end 171.45 125.73) (width 0.254) (layer F.Cu) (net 22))
 (segment (start 175.462727 129.107727) (end 172.085 125.73) (width 0.254) (layer F.Cu) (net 22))
 (segment (start 174.907318 129.671687) (end 174.883687 129.671687) (width 0.254) (layer F.Cu) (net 21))
 (segment (start 170.434 127.254) (end 168.91 125.73) (width 0.254) (layer F.Cu) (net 21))
 (segment (start 172.466 127.254) (end 170.434 127.254) (width 0.254) (layer F.Cu) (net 21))
 (segment (start 174.883687 129.671687) (end 172.466 127.254) (width 0.254) (layer F.Cu) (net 21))
 (segment (start 174.339766 130.239239) (end 174.308239 130.239239) (width 0.254) (layer F.Cu) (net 20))
 (segment (start 168.529 127.889) (end 166.37 125.73) (width 0.254) (layer F.Cu) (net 20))
 (segment (start 171.958 127.889) (end 168.529 127.889) (width 0.254) (layer F.Cu) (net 20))
 (segment (start 174.308239 130.239239) (end 171.958 127.889) (width 0.254) (layer F.Cu) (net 20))
 (segment (start 173.775806 130.803199) (end 173.729199 130.803199) (width 0.254) (layer F.Cu) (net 19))
 (segment (start 166.624 128.524) (end 163.83 125.73) (width 0.254) (layer F.Cu) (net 19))
 (segment (start 171.45 128.524) (end 166.624 128.524) (width 0.254) (layer F.Cu) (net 19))
 (segment (start 173.729199 130.803199) (end 171.45 128.524) (width 0.254) (layer F.Cu) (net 19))
 (segment (start 172.651478 134.758104) (end 172.581896 134.758104) (width 0.254) (layer F.Cu) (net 8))
 (segment (start 163.195 136.525) (end 158.75 140.97) (width 0.254) (layer F.Cu) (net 8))
 (segment (start 170.815 136.525) (end 163.195 136.525) (width 0.254) (layer F.Cu) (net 8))
 (segment (start 172.581896 134.758104) (end 170.815 136.525) (width 0.254) (layer F.Cu) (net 8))
 (segment (start 173.78299 135.889616) (end 173.736384 135.889616) (width 0.254) (layer F.Cu) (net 6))
 (segment (start 166.751 138.049) (end 163.83 140.97) (width 0.254) (layer F.Cu) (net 6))
 (segment (start 171.577 138.049) (end 166.751 138.049) (width 0.254) (layer F.Cu) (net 6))
 (segment (start 173.736384 135.889616) (end 171.577 138.049) (width 0.254) (layer F.Cu) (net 6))
 (segment (start 164.338 120.5865) (end 168.0845 120.5865) (width 0.254) (layer F.Cu) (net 35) (status 20))
 (segment (start 168.0845 120.5865) (end 168.402 120.269) (width 0.254) (layer F.Cu) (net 35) (status 30))
 (segment (start 159.258 118.237) (end 162.687 118.237) (width 0.254) (layer F.Cu) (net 34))
 (segment (start 163.1315 118.6815) (end 164.338 118.6815) (width 0.254) (layer F.Cu) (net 34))
 (segment (start 162.687 118.237) (end 163.1315 118.6815) (width 0.254) (layer F.Cu) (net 34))
 (segment (start 181.107287 129.686056) (end 181.336944 129.686056) (width 0.254) (layer F.Cu) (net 14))
 (segment (start 185.293 127.127) (end 186.69 125.73) (width 0.254) (layer F.Cu) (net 14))
 (segment (start 183.896 127.127) (end 185.293 127.127) (width 0.254) (layer F.Cu) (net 14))
 (segment (start 181.336944 129.686056) (end 183.896 127.127) (width 0.254) (layer F.Cu) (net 14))
 (segment (start 173.217234 135.32386) (end 173.15914 135.32386) (width 0.254) (layer F.Cu) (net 7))
 (segment (start 164.973 137.287) (end 161.29 140.97) (width 0.254) (layer F.Cu) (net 7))
 (segment (start 171.196 137.287) (end 164.973 137.287) (width 0.254) (layer F.Cu) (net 7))
 (segment (start 173.15914 135.32386) (end 171.196 137.287) (width 0.254) (layer F.Cu) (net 7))
 (segment (start 174.348746 136.455373) (end 174.313627 136.455373) (width 0.254) (layer F.Cu) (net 5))
 (segment (start 168.529 138.811) (end 166.37 140.97) (width 0.254) (layer F.Cu) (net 5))
 (segment (start 171.958 138.811) (end 168.529 138.811) (width 0.254) (layer F.Cu) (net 5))
 (segment (start 174.313627 136.455373) (end 171.958 138.811) (width 0.254) (layer F.Cu) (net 5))
 (segment (start 174.914502 137.021129) (end 174.890871 137.021129) (width 0.254) (layer F.Cu) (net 4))
 (segment (start 170.434 139.446) (end 168.91 140.97) (width 0.254) (layer F.Cu) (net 4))
 (segment (start 172.466 139.446) (end 170.434 139.446) (width 0.254) (layer F.Cu) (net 4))
 (segment (start 174.890871 137.021129) (end 172.466 139.446) (width 0.254) (layer F.Cu) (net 4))
 (segment (start 175.480259 137.586885) (end 175.468115 137.586885) (width 0.254) (layer F.Cu) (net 3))
 (segment (start 172.085 140.97) (end 171.45 140.97) (width 0.254) (layer F.Cu) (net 3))
 (segment (start 175.468115 137.586885) (end 172.085 140.97) (width 0.254) (layer F.Cu) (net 3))
 (segment (start 179.975775 128.554543) (end 180.055457 128.554543) (width 0.254) (layer F.Cu) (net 16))
 (segment (start 181.61 127) (end 181.61 125.73) (width 0.254) (layer F.Cu) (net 16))
 (segment (start 180.055457 128.554543) (end 181.61 127) (width 0.254) (layer F.Cu) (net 16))
 (segment (start 176.046015 138.152641) (end 176.045359 138.152641) (width 0.254) (layer F.Cu) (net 2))
 (segment (start 173.99 140.208) (end 173.99 140.97) (width 0.254) (layer F.Cu) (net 2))
 (segment (start 176.045359 138.152641) (end 173.99 140.208) (width 0.254) (layer F.Cu) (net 2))
 (segment (start 176.611771 138.718397) (end 176.611771 140.888229) (width 0.254) (layer F.Cu) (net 1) (status 10))
 (segment (start 176.611771 140.888229) (end 176.53 140.97) (width 0.254) (layer F.Cu) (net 1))
 (segment (start 168.402 118.745) (end 166.624 118.745) (width 0.254) (layer F.Cu) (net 33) (status 10))
 (segment (start 161.671 121.539) (end 159.258 121.539) (width 0.254) (layer F.Cu) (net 33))
 (via (at 161.671 121.539) (size 0.6096) (drill 0.3048) (layers F.Cu B.Cu) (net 33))
 (segment (start 163.449 119.761) (end 161.671 121.539) (width 0.254) (layer B.Cu) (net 33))
 (segment (start 165.608 119.761) (end 163.449 119.761) (width 0.254) (layer B.Cu) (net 33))
 (segment (start 166.624 118.745) (end 165.608 119.761) (width 0.254) (layer B.Cu) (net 33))
 (via (at 166.624 118.745) (size 0.6096) (drill 0.3048) (layers F.Cu B.Cu) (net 33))
 (segment (start 179.418999 127.997767) (end 179.418999 126.078999) (width 0.254) (layer F.Cu) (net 9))
 (segment (start 179.418999 126.078999) (end 179.07 125.73) (width 0.254) (layer F.Cu) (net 9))
 (segment (start 176.602791 127.976215) (end 176.602791 125.802791) (width 0.254) (layer F.Cu) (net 24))
 (segment (start 176.602791 125.802791) (end 176.53 125.73) (width 0.254) (layer F.Cu) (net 24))
 (segment (start 181.682023 136.475129) (end 181.687129 136.475129) (width 0.254) (layer F.Cu) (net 29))
 (segment (start 187.198 138.938) (end 189.23 140.97) (width 0.254) (layer F.Cu) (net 29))
 (segment (start 184.15 138.938) (end 187.198 138.938) (width 0.254) (layer F.Cu) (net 29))
 (segment (start 181.687129 136.475129) (end 184.15 138.938) (width 0.254) (layer F.Cu) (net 29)))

